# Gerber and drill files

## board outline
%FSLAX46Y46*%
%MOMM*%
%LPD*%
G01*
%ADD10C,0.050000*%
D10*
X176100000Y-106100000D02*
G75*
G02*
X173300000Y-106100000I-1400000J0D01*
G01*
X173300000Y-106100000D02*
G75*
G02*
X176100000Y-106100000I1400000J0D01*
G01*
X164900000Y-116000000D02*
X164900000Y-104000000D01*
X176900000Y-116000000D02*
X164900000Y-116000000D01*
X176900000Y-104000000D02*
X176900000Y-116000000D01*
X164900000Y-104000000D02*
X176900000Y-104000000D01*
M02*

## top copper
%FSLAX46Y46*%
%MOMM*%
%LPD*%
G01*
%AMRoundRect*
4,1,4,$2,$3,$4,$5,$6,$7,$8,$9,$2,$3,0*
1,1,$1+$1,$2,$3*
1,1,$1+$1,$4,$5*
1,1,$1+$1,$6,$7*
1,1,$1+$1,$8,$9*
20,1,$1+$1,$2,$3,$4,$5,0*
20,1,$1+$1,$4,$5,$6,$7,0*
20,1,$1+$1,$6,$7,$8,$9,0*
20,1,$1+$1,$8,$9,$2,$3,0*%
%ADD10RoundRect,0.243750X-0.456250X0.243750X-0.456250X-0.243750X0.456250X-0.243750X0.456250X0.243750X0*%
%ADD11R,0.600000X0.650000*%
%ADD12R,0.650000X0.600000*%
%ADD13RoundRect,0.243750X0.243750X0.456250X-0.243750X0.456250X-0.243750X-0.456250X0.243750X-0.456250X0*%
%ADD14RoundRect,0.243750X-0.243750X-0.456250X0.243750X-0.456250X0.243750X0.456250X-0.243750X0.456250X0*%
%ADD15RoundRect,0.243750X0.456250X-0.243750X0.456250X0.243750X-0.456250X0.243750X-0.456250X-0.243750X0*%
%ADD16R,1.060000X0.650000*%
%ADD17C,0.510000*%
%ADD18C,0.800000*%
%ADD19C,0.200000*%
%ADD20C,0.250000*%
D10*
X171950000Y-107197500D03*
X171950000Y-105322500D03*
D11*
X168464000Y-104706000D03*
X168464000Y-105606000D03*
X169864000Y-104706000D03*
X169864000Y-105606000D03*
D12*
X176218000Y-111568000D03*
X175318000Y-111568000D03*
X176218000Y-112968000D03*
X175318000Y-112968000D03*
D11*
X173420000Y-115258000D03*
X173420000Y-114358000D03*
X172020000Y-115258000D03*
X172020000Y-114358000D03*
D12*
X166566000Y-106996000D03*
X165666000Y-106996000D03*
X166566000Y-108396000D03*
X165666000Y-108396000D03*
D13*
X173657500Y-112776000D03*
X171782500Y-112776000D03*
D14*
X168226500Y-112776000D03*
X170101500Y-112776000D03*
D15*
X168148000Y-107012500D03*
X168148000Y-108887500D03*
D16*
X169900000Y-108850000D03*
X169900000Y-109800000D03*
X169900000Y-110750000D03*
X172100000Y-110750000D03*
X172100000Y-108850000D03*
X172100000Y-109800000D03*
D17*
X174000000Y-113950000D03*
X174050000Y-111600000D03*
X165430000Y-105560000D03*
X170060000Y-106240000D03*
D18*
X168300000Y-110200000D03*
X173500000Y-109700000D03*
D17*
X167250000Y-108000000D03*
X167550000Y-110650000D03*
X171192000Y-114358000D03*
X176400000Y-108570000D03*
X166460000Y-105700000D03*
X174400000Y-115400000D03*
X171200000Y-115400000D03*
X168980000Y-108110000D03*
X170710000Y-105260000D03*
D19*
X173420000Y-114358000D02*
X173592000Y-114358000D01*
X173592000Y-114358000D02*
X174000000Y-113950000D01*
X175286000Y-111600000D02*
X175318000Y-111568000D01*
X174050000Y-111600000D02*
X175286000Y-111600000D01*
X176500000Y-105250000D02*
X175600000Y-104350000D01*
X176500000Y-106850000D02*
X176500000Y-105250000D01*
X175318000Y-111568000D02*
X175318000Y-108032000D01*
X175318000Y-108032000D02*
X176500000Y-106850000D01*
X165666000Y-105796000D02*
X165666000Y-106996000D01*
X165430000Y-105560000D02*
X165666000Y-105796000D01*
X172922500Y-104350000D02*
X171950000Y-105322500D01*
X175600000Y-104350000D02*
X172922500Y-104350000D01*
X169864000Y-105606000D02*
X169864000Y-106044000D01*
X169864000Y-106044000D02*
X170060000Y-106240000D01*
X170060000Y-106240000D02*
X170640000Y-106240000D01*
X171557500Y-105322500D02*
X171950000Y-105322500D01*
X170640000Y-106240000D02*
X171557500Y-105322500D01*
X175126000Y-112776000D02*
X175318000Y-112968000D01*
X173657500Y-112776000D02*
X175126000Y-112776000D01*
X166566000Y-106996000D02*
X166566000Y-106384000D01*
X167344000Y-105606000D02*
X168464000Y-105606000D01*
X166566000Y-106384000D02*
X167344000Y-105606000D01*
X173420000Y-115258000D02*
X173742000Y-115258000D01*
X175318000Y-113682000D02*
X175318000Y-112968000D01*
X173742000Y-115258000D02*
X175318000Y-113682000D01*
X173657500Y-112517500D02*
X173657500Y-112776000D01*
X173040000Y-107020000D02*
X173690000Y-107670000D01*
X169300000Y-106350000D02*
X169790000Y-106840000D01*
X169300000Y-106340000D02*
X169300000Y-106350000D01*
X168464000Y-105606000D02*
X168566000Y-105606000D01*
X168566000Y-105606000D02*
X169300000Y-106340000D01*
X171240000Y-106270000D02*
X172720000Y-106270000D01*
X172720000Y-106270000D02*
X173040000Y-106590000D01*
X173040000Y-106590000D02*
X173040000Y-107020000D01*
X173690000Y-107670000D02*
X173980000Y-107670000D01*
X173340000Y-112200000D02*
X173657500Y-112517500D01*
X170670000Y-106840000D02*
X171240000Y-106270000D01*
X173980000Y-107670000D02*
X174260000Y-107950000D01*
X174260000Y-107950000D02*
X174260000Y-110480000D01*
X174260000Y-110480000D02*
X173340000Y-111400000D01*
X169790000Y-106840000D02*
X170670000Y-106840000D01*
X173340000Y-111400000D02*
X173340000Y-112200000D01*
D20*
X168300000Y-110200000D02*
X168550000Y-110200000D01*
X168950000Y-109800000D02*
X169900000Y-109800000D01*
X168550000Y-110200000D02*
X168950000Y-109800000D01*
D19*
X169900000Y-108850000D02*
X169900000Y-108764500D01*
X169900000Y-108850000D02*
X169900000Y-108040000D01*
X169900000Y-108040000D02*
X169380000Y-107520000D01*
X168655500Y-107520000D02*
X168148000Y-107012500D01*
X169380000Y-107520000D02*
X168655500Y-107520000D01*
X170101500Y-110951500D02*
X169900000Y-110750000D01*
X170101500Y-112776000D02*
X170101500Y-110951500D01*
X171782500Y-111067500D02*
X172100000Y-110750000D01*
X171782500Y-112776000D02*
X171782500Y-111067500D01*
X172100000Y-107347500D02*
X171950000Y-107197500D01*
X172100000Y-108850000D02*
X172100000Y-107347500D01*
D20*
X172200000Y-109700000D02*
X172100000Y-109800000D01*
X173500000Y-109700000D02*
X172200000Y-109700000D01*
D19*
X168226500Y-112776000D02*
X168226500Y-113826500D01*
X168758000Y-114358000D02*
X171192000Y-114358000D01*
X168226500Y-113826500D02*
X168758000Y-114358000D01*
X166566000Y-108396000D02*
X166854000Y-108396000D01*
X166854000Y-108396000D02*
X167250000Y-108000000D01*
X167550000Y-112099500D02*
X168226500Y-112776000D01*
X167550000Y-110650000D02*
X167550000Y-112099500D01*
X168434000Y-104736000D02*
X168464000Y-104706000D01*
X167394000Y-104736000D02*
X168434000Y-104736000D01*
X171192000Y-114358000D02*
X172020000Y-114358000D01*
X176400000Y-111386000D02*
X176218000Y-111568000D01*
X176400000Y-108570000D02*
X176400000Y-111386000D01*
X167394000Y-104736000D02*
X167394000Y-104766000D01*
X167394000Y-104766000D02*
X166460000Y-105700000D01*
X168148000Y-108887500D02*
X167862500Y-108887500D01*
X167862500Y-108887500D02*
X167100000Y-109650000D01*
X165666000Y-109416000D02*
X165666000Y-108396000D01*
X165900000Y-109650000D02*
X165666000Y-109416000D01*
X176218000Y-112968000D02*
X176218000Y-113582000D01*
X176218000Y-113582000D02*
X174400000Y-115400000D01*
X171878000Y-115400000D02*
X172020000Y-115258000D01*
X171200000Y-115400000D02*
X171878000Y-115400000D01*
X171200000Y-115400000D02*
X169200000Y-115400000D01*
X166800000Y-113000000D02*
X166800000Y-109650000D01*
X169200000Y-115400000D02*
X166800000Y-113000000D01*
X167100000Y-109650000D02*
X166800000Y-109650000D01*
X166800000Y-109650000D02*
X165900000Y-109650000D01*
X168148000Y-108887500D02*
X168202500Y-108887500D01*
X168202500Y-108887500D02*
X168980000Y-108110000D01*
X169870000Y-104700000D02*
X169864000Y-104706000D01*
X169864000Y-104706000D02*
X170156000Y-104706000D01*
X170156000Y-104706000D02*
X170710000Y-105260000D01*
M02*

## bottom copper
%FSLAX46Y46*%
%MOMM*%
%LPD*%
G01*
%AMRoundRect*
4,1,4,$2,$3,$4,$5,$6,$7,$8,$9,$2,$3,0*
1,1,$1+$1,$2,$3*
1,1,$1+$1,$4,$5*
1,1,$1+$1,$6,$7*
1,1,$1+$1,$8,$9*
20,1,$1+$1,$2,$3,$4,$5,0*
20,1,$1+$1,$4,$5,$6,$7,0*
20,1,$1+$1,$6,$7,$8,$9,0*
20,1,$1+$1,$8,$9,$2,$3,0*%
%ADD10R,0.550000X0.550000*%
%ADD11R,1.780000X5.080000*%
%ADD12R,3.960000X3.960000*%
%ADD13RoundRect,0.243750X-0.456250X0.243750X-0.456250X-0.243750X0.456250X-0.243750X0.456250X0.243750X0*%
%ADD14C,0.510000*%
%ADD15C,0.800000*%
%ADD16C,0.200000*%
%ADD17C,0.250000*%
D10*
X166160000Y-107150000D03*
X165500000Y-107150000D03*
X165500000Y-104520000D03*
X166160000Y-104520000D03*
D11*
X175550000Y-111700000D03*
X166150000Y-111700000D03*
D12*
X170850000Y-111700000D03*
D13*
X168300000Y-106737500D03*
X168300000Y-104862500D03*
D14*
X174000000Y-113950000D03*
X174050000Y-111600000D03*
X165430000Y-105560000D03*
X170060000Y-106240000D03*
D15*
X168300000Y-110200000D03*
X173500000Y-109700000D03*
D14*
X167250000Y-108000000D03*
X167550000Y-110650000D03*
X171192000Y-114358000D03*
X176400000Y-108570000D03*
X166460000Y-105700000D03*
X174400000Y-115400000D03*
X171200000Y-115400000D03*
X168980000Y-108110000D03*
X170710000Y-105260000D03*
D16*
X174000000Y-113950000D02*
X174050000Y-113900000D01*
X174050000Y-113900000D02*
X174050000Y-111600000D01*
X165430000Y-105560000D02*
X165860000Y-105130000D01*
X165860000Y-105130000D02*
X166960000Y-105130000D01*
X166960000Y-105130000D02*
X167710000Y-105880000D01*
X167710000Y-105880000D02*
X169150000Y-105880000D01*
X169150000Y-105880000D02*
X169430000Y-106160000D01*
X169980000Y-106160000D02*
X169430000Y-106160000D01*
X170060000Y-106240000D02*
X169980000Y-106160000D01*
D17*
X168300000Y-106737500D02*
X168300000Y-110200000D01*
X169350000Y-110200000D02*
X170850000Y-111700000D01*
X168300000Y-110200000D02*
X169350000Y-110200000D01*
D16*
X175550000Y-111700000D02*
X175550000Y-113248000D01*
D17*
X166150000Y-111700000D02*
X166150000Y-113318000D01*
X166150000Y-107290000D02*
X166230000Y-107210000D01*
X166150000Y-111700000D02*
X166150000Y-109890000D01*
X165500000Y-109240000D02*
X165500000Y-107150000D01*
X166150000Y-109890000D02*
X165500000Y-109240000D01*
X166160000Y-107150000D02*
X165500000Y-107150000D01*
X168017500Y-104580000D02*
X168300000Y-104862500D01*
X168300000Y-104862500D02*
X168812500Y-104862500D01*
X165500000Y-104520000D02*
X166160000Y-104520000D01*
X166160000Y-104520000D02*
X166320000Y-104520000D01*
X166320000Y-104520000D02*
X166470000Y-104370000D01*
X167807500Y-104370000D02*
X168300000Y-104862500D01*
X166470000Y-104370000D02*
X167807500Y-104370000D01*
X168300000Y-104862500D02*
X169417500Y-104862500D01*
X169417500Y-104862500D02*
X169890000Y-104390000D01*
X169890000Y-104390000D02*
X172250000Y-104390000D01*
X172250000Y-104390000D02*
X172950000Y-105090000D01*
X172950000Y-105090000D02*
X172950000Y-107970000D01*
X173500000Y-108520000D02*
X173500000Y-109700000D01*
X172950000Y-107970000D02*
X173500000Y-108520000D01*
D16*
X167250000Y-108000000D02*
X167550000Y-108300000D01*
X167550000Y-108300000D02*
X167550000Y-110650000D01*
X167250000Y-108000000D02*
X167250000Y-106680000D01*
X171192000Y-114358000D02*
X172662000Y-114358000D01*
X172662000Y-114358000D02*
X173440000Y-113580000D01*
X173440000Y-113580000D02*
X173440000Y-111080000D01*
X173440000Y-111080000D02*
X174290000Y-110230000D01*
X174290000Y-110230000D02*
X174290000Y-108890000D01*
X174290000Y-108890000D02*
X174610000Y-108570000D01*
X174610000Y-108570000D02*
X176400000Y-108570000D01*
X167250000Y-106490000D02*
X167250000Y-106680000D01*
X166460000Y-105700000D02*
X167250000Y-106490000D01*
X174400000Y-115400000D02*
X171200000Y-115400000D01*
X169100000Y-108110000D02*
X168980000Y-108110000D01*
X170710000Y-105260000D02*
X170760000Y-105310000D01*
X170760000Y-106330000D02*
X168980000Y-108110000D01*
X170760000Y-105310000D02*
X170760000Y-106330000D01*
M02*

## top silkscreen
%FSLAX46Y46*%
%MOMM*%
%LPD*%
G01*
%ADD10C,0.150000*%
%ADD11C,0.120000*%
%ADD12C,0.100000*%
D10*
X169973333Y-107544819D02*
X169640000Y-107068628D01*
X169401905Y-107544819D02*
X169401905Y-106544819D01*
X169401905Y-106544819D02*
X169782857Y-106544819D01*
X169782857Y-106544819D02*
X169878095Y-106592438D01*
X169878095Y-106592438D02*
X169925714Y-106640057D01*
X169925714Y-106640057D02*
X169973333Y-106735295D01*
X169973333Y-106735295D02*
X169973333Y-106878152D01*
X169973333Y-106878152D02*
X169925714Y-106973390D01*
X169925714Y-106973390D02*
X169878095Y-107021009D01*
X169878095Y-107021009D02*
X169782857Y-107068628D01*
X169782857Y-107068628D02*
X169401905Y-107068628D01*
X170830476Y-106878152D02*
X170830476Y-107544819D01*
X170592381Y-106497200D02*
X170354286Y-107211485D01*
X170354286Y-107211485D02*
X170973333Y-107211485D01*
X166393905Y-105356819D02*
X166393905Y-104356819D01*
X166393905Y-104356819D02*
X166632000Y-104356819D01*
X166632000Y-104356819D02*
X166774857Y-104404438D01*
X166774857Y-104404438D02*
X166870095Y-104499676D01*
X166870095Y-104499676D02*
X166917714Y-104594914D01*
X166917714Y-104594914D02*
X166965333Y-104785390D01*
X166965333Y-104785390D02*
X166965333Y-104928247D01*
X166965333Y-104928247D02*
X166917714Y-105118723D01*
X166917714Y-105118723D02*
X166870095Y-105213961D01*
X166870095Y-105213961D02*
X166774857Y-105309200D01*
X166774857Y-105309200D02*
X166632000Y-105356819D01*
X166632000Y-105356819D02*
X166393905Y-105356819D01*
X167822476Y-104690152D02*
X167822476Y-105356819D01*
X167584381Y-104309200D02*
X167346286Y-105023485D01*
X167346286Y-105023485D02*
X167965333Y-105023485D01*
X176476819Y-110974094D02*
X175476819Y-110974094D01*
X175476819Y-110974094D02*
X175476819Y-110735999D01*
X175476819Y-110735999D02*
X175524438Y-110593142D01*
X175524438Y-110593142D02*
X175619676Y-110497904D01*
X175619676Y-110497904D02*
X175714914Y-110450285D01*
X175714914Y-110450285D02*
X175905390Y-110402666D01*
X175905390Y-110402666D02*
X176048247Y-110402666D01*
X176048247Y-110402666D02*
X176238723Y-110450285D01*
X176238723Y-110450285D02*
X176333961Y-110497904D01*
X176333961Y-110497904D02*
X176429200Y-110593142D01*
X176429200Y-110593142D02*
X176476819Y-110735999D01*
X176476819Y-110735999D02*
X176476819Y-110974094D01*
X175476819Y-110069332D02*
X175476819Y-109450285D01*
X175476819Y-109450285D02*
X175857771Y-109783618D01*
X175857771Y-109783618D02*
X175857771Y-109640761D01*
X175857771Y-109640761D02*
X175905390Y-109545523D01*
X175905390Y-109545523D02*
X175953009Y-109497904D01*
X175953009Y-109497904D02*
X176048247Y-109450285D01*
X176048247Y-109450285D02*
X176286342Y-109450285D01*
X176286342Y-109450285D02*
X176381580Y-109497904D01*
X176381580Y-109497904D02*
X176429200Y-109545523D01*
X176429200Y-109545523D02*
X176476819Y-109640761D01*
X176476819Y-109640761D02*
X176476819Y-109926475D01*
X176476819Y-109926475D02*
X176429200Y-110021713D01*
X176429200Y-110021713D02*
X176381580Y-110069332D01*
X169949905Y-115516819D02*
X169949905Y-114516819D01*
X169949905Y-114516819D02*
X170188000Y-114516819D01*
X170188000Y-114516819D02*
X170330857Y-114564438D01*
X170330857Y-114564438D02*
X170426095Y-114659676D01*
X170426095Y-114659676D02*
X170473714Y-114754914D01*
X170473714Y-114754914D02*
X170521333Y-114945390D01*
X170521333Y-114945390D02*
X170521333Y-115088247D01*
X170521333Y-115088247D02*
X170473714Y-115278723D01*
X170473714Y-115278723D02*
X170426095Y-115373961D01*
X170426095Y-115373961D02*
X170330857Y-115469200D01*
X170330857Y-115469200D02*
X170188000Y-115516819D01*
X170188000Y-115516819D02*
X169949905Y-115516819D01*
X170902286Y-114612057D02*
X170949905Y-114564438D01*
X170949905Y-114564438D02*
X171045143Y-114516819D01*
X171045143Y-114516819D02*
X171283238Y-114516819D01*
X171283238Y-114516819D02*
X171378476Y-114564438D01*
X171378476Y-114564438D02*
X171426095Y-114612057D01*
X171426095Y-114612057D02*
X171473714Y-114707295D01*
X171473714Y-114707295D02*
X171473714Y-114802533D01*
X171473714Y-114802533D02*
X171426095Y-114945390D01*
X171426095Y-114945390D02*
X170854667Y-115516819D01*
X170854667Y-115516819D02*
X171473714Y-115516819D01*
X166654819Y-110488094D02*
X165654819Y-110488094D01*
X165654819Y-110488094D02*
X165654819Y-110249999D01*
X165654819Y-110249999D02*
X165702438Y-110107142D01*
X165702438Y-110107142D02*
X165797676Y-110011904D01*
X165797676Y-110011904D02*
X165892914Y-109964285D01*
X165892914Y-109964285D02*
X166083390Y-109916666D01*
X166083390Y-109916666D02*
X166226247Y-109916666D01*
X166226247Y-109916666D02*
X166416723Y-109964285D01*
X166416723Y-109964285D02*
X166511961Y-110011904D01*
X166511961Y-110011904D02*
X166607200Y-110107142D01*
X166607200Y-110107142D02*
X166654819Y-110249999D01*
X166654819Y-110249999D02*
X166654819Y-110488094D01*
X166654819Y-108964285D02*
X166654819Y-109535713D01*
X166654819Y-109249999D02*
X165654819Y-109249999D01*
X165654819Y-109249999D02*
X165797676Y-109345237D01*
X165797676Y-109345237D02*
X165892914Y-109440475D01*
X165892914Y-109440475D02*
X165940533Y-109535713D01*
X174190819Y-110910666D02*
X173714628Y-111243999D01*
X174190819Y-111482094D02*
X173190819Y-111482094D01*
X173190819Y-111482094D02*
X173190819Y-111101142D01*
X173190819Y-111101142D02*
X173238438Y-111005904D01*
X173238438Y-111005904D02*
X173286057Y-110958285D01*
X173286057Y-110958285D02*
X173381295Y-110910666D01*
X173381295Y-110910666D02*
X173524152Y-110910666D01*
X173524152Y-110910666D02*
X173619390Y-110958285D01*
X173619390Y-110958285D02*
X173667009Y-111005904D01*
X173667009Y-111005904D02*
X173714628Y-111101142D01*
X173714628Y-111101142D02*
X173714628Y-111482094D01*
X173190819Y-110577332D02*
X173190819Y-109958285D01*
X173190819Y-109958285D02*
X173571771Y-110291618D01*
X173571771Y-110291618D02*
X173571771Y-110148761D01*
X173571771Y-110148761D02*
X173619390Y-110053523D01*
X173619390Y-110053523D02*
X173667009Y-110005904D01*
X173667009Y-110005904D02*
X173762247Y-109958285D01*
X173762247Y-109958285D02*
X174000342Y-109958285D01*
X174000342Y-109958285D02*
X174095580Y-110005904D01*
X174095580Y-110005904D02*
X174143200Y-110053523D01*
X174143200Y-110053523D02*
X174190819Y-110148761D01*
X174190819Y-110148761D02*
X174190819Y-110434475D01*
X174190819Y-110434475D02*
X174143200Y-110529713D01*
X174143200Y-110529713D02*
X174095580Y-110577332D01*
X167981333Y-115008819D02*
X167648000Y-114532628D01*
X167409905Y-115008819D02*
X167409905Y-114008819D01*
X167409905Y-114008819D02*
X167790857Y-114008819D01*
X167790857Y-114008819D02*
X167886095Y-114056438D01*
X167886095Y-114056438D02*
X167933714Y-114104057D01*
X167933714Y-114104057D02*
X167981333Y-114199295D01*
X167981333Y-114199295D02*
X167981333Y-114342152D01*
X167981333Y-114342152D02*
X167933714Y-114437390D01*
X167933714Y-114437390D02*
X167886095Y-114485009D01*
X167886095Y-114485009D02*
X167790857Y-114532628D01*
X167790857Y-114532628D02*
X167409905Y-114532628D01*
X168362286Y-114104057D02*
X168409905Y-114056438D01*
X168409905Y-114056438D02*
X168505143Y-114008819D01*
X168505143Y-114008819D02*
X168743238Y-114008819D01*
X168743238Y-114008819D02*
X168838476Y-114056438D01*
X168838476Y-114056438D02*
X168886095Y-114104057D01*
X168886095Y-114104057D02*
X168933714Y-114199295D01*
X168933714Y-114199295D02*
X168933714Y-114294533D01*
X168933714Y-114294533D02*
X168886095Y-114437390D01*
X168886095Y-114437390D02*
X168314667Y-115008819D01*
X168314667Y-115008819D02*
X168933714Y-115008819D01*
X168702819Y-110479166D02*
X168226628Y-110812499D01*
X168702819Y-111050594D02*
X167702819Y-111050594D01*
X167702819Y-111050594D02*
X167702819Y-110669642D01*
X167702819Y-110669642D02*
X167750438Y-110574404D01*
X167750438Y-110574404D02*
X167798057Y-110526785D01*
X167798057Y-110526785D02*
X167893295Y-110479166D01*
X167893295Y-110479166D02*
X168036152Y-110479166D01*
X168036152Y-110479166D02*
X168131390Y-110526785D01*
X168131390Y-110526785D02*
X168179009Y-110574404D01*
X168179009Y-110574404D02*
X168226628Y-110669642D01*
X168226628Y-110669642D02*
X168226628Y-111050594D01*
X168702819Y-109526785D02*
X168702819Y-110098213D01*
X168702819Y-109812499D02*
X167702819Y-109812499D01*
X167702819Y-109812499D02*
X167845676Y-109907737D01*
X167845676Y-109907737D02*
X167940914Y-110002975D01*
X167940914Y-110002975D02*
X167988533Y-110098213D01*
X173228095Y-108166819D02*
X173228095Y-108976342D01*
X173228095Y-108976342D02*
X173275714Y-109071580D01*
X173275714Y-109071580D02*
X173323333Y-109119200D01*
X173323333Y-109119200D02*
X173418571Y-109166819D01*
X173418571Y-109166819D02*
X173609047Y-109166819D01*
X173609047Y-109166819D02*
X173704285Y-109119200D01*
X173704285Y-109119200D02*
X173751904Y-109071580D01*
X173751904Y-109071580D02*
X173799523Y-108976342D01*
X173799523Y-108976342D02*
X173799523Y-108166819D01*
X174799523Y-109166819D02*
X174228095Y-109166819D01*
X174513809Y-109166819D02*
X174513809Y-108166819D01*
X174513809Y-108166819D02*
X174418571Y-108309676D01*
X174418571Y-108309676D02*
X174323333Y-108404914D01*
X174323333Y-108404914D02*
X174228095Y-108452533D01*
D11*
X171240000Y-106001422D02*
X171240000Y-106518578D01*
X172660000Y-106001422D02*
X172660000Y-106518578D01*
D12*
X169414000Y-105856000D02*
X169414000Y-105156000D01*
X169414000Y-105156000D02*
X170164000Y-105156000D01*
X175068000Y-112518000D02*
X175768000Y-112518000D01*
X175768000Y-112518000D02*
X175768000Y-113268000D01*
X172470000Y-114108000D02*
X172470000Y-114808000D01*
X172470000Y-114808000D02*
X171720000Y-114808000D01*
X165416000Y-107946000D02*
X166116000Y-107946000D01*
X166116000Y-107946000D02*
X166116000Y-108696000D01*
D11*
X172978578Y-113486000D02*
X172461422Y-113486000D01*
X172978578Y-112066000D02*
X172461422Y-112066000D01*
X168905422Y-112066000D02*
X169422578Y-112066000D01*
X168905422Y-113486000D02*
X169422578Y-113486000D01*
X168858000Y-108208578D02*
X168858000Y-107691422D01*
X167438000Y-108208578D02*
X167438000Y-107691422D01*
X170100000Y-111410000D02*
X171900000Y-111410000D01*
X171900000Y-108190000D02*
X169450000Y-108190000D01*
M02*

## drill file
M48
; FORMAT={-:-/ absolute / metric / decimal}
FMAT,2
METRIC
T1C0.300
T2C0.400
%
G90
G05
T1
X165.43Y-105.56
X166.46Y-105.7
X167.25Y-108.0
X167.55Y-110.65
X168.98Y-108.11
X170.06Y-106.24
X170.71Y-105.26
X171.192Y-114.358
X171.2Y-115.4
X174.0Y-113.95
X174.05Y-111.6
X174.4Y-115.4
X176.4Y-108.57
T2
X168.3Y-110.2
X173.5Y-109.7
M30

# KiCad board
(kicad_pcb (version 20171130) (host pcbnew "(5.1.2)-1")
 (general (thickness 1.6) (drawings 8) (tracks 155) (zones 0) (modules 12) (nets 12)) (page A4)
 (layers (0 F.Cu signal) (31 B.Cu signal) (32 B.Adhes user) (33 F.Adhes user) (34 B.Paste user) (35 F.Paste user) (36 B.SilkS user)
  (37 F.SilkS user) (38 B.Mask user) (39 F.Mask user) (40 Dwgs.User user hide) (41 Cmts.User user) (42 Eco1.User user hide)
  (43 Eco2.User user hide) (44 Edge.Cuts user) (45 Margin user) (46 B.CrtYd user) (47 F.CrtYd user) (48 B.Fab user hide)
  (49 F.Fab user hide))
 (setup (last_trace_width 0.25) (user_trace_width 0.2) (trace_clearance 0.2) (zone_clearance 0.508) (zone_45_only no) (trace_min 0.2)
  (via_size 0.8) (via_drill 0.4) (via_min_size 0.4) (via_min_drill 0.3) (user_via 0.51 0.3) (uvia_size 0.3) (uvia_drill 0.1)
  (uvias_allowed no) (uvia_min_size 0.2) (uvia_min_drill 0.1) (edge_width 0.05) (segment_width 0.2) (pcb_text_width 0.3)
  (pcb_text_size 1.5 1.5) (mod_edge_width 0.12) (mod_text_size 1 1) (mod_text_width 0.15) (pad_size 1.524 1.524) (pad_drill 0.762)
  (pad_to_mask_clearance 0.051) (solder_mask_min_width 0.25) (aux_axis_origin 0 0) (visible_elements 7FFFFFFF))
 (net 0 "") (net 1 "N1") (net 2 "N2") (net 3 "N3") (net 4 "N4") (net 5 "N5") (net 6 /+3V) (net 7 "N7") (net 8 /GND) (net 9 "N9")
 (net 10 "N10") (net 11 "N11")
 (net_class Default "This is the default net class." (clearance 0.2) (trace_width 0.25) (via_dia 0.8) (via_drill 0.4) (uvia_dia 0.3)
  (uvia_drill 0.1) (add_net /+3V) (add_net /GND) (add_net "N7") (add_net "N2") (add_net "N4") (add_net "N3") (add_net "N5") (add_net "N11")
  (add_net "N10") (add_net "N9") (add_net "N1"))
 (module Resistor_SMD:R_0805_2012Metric (layer F.Cu) (at 171.95 106.26 270)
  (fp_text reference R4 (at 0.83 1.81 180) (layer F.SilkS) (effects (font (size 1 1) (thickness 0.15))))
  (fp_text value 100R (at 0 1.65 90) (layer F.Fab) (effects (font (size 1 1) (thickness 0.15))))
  (fp_line (start -0.258578 0.71) (end 0.258578 0.71) (layer F.SilkS) (width 0.12))
  (fp_line (start -0.258578 -0.71) (end 0.258578 -0.71) (layer F.SilkS) (width 0.12))
  (pad 2 smd roundrect (at 0.9375 0 270) (size 0.975 1.4) (layers F.Cu F.Paste F.Mask) (roundrect_rratio 0.25) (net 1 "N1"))
  (pad 1 smd roundrect (at -0.9375 0 270) (size 0.975 1.4) (layers F.Cu F.Paste F.Mask) (roundrect_rratio 0.25) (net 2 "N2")))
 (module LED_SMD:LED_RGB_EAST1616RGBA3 (layer F.Cu) (at 169.164 105.156)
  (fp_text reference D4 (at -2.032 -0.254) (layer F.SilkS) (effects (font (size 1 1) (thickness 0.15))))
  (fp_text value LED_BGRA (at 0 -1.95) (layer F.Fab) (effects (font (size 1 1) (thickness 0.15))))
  (fp_line (start 0.25 0.7) (end 0.25 0) (layer F.SilkS) (width 0.1))
  (fp_line (start 0.25 0) (end 1 0) (layer F.SilkS) (width 0.1))
  (pad 2 smd rect (at -0.7 -0.45) (size 0.6 0.65) (layers F.Cu F.Paste F.Mask) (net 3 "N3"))
  (pad 1 smd rect (at -0.7 0.45) (size 0.6 0.65) (layers F.Cu F.Paste F.Mask) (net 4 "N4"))
  (pad 3 smd rect (at 0.7 -0.45) (size 0.6 0.65) (layers F.Cu F.Paste F.Mask) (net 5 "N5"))
  (pad 4 smd rect (at 0.7 0.45) (size 0.6 0.65) (layers F.Cu F.Paste F.Mask) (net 2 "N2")))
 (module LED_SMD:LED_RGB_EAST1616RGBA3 (layer F.Cu) (at 175.768 112.268 270)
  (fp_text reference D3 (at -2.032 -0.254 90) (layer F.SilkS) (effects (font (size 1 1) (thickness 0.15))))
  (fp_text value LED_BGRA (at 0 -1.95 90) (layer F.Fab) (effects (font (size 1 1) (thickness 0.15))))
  (fp_line (start 0.25 0.7) (end 0.25 0) (layer F.SilkS) (width 0.1))
  (fp_line (start 0.25 0) (end 1 0) (layer F.SilkS) (width 0.1))
  (pad 2 smd rect (at -0.7 -0.45 270) (size 0.6 0.65) (layers F.Cu F.Paste F.Mask) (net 3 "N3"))
  (pad 1 smd rect (at -0.7 0.45 270) (size 0.6 0.65) (layers F.Cu F.Paste F.Mask) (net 2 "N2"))
  (pad 3 smd rect (at 0.7 -0.45 270) (size 0.6 0.65) (layers F.Cu F.Paste F.Mask) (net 5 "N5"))
  (pad 4 smd rect (at 0.7 0.45 270) (size 0.6 0.65) (layers F.Cu F.Paste F.Mask) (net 4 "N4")))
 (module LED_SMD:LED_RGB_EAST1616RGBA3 (layer F.Cu) (at 172.72 114.808 180)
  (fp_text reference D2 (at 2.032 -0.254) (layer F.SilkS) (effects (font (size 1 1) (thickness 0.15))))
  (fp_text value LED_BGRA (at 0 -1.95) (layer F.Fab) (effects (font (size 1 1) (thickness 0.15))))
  (fp_line (start 0.25 0.7) (end 0.25 0) (layer F.SilkS) (width 0.1))
  (fp_line (start 0.25 0) (end 1 0) (layer F.SilkS) (width 0.1))
  (pad 2 smd rect (at -0.7 -0.45 180) (size 0.6 0.65) (layers F.Cu F.Paste F.Mask) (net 4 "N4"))
  (pad 1 smd rect (at -0.7 0.45 180) (size 0.6 0.65) (layers F.Cu F.Paste F.Mask) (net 2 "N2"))
  (pad 3 smd rect (at 0.7 -0.45 180) (size 0.6 0.65) (layers F.Cu F.Paste F.Mask) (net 5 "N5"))
  (pad 4 smd rect (at 0.7 0.45 180) (size 0.6 0.65) (layers F.Cu F.Paste F.Mask) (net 3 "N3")))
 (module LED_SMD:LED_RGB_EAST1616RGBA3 (layer F.Cu) (at 166.116 107.696 270)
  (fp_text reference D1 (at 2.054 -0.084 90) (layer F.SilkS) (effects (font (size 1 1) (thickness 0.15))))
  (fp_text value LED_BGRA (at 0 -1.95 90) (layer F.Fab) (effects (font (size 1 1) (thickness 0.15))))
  (fp_line (start 0.25 0.7) (end 0.25 0) (layer F.SilkS) (width 0.1))
  (fp_line (start 0.25 0) (end 1 0) (layer F.SilkS) (width 0.1))
  (pad 2 smd rect (at -0.7 -0.45 270) (size 0.6 0.65) (layers F.Cu F.Paste F.Mask) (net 4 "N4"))
  (pad 1 smd rect (at -0.7 0.45 270) (size 0.6 0.65) (layers F.Cu F.Paste F.Mask) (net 2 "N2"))
  (pad 3 smd rect (at 0.7 -0.45 270) (size 0.6 0.65) (layers F.Cu F.Paste F.Mask) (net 3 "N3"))
  (pad 4 smd rect (at 0.7 0.45 270) (size 0.6 0.65) (layers F.Cu F.Paste F.Mask) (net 5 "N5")))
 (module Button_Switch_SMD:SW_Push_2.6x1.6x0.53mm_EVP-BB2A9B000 (layer B.Cu) (at 165.83 105.84 90)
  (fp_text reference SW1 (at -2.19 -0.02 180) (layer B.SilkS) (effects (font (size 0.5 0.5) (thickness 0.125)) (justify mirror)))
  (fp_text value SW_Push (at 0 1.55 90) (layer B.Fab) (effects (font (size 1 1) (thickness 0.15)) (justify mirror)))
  (pad 1 smd rect (at -1.31 0.33 90) (size 0.55 0.55) (layers B.Cu B.Paste B.Mask) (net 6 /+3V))
  (pad 1 smd rect (at -1.31 -0.33 90) (size 0.55 0.55) (layers B.Cu B.Paste B.Mask) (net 6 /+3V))
  (pad 2 smd rect (at 1.32 -0.33 90) (size 0.55 0.55) (layers B.Cu B.Paste B.Mask) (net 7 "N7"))
  (pad 2 smd rect (at 1.32 0.33 90) (size 0.55 0.55) (layers B.Cu B.Paste B.Mask) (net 7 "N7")))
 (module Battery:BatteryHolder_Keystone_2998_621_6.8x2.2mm (layer B.Cu) (at 170.85 111.7)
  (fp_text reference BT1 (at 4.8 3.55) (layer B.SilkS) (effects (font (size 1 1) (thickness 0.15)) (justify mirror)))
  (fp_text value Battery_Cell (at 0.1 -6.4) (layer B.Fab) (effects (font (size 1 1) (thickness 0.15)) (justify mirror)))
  (pad 1 smd rect (at 4.7 0) (size 1.78 5.08) (layers B.Cu B.Paste B.Mask) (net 6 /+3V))
  (pad 1 smd rect (at -4.7 0) (size 1.78 5.08) (layers B.Cu B.Paste B.Mask) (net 6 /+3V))
  (pad 2 smd rect (at 0 0) (size 3.96 3.96) (layers B.Cu B.Paste B.Mask) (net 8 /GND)))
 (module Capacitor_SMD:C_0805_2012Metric (layer B.Cu) (at 168.3 105.8 270)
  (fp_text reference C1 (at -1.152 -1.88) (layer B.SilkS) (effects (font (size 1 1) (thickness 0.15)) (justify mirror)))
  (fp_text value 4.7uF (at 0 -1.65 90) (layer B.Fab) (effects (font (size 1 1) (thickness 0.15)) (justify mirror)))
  (pad 2 smd roundrect (at 0.9375 0 270) (size 0.975 1.4) (layers B.Cu B.Paste B.Mask) (roundrect_rratio 0.25) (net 8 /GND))
  (pad 1 smd roundrect (at -0.9375 0 270) (size 0.975 1.4) (layers B.Cu B.Paste B.Mask) (roundrect_rratio 0.25) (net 7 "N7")))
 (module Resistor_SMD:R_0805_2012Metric (layer F.Cu) (at 172.72 112.776 180)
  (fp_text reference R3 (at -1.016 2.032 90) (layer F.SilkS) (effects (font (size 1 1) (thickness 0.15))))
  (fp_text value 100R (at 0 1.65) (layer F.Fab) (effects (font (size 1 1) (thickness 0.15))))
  (fp_line (start -0.258578 -0.71) (end 0.258578 -0.71) (layer F.SilkS) (width 0.12))
  (fp_line (start -0.258578 0.71) (end 0.258578 0.71) (layer F.SilkS) (width 0.12))
  (pad 1 smd roundrect (at -0.9375 0 180) (size 0.975 1.4) (layers F.Cu F.Paste F.Mask) (roundrect_rratio 0.25) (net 4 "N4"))
  (pad 2 smd roundrect (at 0.9375 0 180) (size 0.975 1.4) (layers F.Cu F.Paste F.Mask) (roundrect_rratio 0.25) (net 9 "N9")))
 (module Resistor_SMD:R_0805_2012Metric (layer F.Cu) (at 169.164 112.776)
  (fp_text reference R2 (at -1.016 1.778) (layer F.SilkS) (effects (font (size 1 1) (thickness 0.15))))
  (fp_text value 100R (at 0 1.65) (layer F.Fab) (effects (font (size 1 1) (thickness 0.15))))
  (fp_line (start -0.258578 -0.71) (end 0.258578 -0.71) (layer F.SilkS) (width 0.12))
  (fp_line (start -0.258578 0.71) (end 0.258578 0.71) (layer F.SilkS) (width 0.12))
  (pad 1 smd roundrect (at -0.9375 0) (size 0.975 1.4) (layers F.Cu F.Paste F.Mask) (roundrect_rratio 0.25) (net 3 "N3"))
  (pad 2 smd roundrect (at 0.9375 0) (size 0.975 1.4) (layers F.Cu F.Paste F.Mask) (roundrect_rratio 0.25) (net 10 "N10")))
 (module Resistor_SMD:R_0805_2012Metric (layer F.Cu) (at 168.148 107.95 90)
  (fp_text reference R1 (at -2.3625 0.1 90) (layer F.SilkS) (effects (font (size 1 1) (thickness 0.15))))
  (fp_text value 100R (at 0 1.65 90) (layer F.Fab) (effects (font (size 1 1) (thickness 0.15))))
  (fp_line (start -0.258578 0.71) (end 0.258578 0.71) (layer F.SilkS) (width 0.12))
  (fp_line (start -0.258578 -0.71) (end 0.258578 -0.71) (layer F.SilkS) (width 0.12))
  (pad 2 smd roundrect (at 0.9375 0 90) (size 0.975 1.4) (layers F.Cu F.Paste F.Mask) (roundrect_rratio 0.25) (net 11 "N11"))
  (pad 1 smd roundrect (at -0.9375 0 90) (size 0.975 1.4) (layers F.Cu F.Paste F.Mask) (roundrect_rratio 0.25) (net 5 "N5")))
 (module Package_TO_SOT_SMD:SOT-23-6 (layer F.Cu) (at 171 109.8)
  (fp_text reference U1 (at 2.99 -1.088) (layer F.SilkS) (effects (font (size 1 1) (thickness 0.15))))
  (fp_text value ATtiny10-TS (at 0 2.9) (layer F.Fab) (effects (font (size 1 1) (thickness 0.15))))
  (fp_line (start -0.9 1.61) (end 0.9 1.61) (layer F.SilkS) (width 0.12))
  (fp_line (start 0.9 -1.61) (end -1.55 -1.61) (layer F.SilkS) (width 0.12))
  (pad 1 smd rect (at -1.1 -0.95) (size 1.06 0.65) (layers F.Cu F.Paste F.Mask) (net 11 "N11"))
  (pad 2 smd rect (at -1.1 0) (size 1.06 0.65) (layers F.Cu F.Paste F.Mask) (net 8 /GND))
  (pad 3 smd rect (at -1.1 0.95) (size 1.06 0.65) (layers F.Cu F.Paste F.Mask) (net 10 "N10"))
  (pad 4 smd rect (at 1.1 0.95) (size 1.06 0.65) (layers F.Cu F.Paste F.Mask) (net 9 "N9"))
  (pad 6 smd rect (at 1.1 -0.95) (size 1.06 0.65) (layers F.Cu F.Paste F.Mask) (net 1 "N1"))
  (pad 5 smd rect (at 1.1 0) (size 1.06 0.65) (layers F.Cu F.Paste F.Mask) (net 7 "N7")))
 (gr_circle (center 174.7 106.1) (end 176.1 106.1) (layer Edge.Cuts) (width 0.05))
 (gr_line (start 164.9 116) (end 164.9 104) (layer Edge.Cuts) (width 0.05))
 (gr_line (start 176.9 116) (end 164.9 116) (layer Edge.Cuts) (width 0.05))
 (gr_line (start 176.9 104) (end 176.9 116) (layer Edge.Cuts) (width 0.05))
 (gr_line (start 164.9 104) (end 176.9 104) (layer Edge.Cuts) (width 0.05))
 (via (at 174 113.95) (size 0.51) (drill 0.3) (layers F.Cu B.Cu) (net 2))
 (segment (start 173.42 114.358) (end 173.592 114.358) (width 0.2) (layer F.Cu) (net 2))
 (segment (start 173.592 114.358) (end 174 113.95) (width 0.2) (layer F.Cu) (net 2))
 (via (at 174.05 111.6) (size 0.51) (drill 0.3) (layers F.Cu B.Cu) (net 2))
 (segment (start 174 113.95) (end 174.05 113.9) (width 0.2) (layer B.Cu) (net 2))
 (segment (start 174.05 113.9) (end 174.05 111.6) (width 0.2) (layer B.Cu) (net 2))
 (segment (start 175.286 111.6) (end 175.318 111.568) (width 0.2) (layer F.Cu) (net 2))
 (segment (start 174.05 111.6) (end 175.286 111.6) (width 0.2) (layer F.Cu) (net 2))
 (segment (start 176.5 105.25) (end 175.6 104.35) (width 0.2) (layer F.Cu) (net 2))
 (segment (start 176.5 106.85) (end 176.5 105.25) (width 0.2) (layer F.Cu) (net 2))
 (segment (start 175.318 111.568) (end 175.318 108.032) (width 0.2) (layer F.Cu) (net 2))
 (segment (start 175.318 108.032) (end 176.5 106.85) (width 0.2) (layer F.Cu) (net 2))
 (via (at 165.43 105.56) (size 0.51) (drill 0.3) (layers F.Cu B.Cu) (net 2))
 (segment (start 165.666 105.796) (end 165.666 106.996) (width 0.2) (layer F.Cu) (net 2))
 (segment (start 165.43 105.56) (end 165.666 105.796) (width 0.2) (layer F.Cu) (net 2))
 (segment (start 172.9225 104.35) (end 171.95 105.3225) (width 0.2) (layer F.Cu) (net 2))
 (segment (start 175.6 104.35) (end 172.9225 104.35) (width 0.2) (layer F.Cu) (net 2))
 (segment (start 165.43 105.56) (end 165.86 105.13) (width 0.2) (layer B.Cu) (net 2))
 (segment (start 165.86 105.13) (end 166.96 105.13) (width 0.2) (layer B.Cu) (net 2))
 (segment (start 166.96 105.13) (end 167.71 105.88) (width 0.2) (layer B.Cu) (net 2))
 (segment (start 167.71 105.88) (end 169.15 105.88) (width 0.2) (layer B.Cu) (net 2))
 (segment (start 169.15 105.88) (end 169.43 106.16) (width 0.2) (layer B.Cu) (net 2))
 (via (at 170.06 106.24) (size 0.51) (drill 0.3) (layers F.Cu B.Cu) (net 2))
 (segment (start 169.864 105.606) (end 169.864 106.044) (width 0.2) (layer F.Cu) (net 2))
 (segment (start 169.864 106.044) (end 170.06 106.24) (width 0.2) (layer F.Cu) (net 2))
 (segment (start 169.98 106.16) (end 169.43 106.16) (width 0.2) (layer B.Cu) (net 2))
 (segment (start 170.06 106.24) (end 169.98 106.16) (width 0.2) (layer B.Cu) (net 2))
 (segment (start 170.06 106.24) (end 170.64 106.24) (width 0.2) (layer F.Cu) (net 2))
 (segment (start 171.5575 105.3225) (end 171.95 105.3225) (width 0.2) (layer F.Cu) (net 2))
 (segment (start 170.64 106.24) (end 171.5575 105.3225) (width 0.2) (layer F.Cu) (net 2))
 (segment (start 175.126 112.776) (end 175.318 112.968) (width 0.2) (layer F.Cu) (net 4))
 (segment (start 173.6575 112.776) (end 175.126 112.776) (width 0.2) (layer F.Cu) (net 4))
 (segment (start 166.566 106.996) (end 166.566 106.384) (width 0.2) (layer F.Cu) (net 4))
 (segment (start 167.344 105.606) (end 168.464 105.606) (width 0.2) (layer F.Cu) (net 4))
 (segment (start 166.566 106.384) (end 167.344 105.606) (width 0.2) (layer F.Cu) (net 4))
 (segment (start 173.42 115.258) (end 173.742 115.258) (width 0.2) (layer F.Cu) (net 4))
 (segment (start 175.318 113.682) (end 175.318 112.968) (width 0.2) (layer F.Cu) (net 4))
 (segment (start 173.742 115.258) (end 175.318 113.682) (width 0.2) (layer F.Cu) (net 4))
 (segment (start 173.6575 112.5175) (end 173.6575 112.776) (width 0.2) (layer F.Cu) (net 4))
 (segment (start 173.04 107.02) (end 173.69 107.67) (width 0.2) (layer F.Cu) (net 4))
 (segment (start 169.3 106.35) (end 169.79 106.84) (width 0.2) (layer F.Cu) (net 4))
 (segment (start 169.3 106.34) (end 169.3 106.35) (width 0.2) (layer F.Cu) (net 4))
 (segment (start 168.464 105.606) (end 168.566 105.606) (width 0.2) (layer F.Cu) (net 4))
 (segment (start 168.566 105.606) (end 169.3 106.34) (width 0.2) (layer F.Cu) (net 4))
 (segment (start 171.24 106.27) (end 172.72 106.27) (width 0.2) (layer F.Cu) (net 4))
 (segment (start 172.72 106.27) (end 173.04 106.59) (width 0.2) (layer F.Cu) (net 4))
 (segment (start 173.04 106.59) (end 173.04 107.02) (width 0.2) (layer F.Cu) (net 4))
 (segment (start 173.69 107.67) (end 173.98 107.67) (width 0.2) (layer F.Cu) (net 4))
 (segment (start 173.34 112.2) (end 173.6575 112.5175) (width 0.2) (layer F.Cu) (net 4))
 (segment (start 170.67 106.84) (end 171.24 106.27) (width 0.2) (layer F.Cu) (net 4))
 (segment (start 173.98 107.67) (end 174.26 107.95) (width 0.2) (layer F.Cu) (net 4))
 (segment (start 174.26 107.95) (end 174.26 110.48) (width 0.2) (layer F.Cu) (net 4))
 (segment (start 174.26 110.48) (end 173.34 111.4) (width 0.2) (layer F.Cu) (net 4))
 (segment (start 169.79 106.84) (end 170.67 106.84) (width 0.2) (layer F.Cu) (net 4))
 (segment (start 173.34 111.4) (end 173.34 112.2) (width 0.2) (layer F.Cu) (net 4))
 (via (at 168.3 110.2) (size 0.8) (drill 0.4) (layers F.Cu B.Cu) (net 8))
 (segment (start 168.3 106.7375) (end 168.3 110.2) (width 0.25) (layer B.Cu) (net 8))
 (segment (start 168.3 110.2) (end 168.55 110.2) (width 0.25) (layer F.Cu) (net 8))
 (segment (start 168.95 109.8) (end 169.9 109.8) (width 0.25) (layer F.Cu) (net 8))
 (segment (start 168.55 110.2) (end 168.95 109.8) (width 0.25) (layer F.Cu) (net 8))
 (segment (start 169.35 110.2) (end 170.85 111.7) (width 0.25) (layer B.Cu) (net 8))
 (segment (start 168.3 110.2) (end 169.35 110.2) (width 0.25) (layer B.Cu) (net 8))
 (segment (start 169.9 108.85) (end 169.9 108.7645) (width 0.2) (layer F.Cu) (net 11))
 (segment (start 169.9 108.85) (end 169.9 108.04) (width 0.2) (layer F.Cu) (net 11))
 (segment (start 169.9 108.04) (end 169.38 107.52) (width 0.2) (layer F.Cu) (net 11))
 (segment (start 168.6555 107.52) (end 168.148 107.0125) (width 0.2) (layer F.Cu) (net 11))
 (segment (start 169.38 107.52) (end 168.6555 107.52) (width 0.2) (layer F.Cu) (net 11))
 (segment (start 170.1015 110.9515) (end 169.9 110.75) (width 0.2) (layer F.Cu) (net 10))
 (segment (start 170.1015 112.776) (end 170.1015 110.9515) (width 0.2) (layer F.Cu) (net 10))
 (segment (start 171.7825 111.0675) (end 172.1 110.75) (width 0.2) (layer F.Cu) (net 9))
 (segment (start 171.7825 112.776) (end 171.7825 111.0675) (width 0.2) (layer F.Cu) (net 9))
 (segment (start 172.1 107.3475) (end 171.95 107.1975) (width 0.2) (layer F.Cu) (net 1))
 (segment (start 172.1 108.85) (end 172.1 107.3475) (width 0.2) (layer F.Cu) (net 1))
 (segment (start 175.55 111.7) (end 175.55 113.248) (width 0.2) (layer B.Cu) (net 6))
 (segment (start 166.15 111.7) (end 166.15 113.318) (width 0.25) (layer B.Cu) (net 6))
 (segment (start 166.15 107.29) (end 166.23 107.21) (width 0.25) (layer B.Cu) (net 6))
 (segment (start 166.15 111.7) (end 166.15 109.89) (width 0.25) (layer B.Cu) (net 6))
 (segment (start 165.5 109.24) (end 165.5 107.15) (width 0.25) (layer B.Cu) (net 6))
 (segment (start 166.15 109.89) (end 165.5 109.24) (width 0.25) (layer B.Cu) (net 6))
 (segment (start 166.16 107.15) (end 165.5 107.15) (width 0.25) (layer B.Cu) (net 6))
 (segment (start 168.0175 104.58) (end 168.3 104.8625) (width 0.25) (layer B.Cu) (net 7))
 (via (at 173.5 109.7) (size 0.8) (drill 0.4) (layers F.Cu B.Cu) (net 7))
 (segment (start 172.2 109.7) (end 172.1 109.8) (width 0.25) (layer F.Cu) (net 7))
 (segment (start 173.5 109.7) (end 172.2 109.7) (width 0.25) (layer F.Cu) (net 7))
 (segment (start 168.3 104.8625) (end 168.8125 104.8625) (width 0.25) (layer B.Cu) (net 7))
 (segment (start 165.5 104.52) (end 166.16 104.52) (width 0.25) (layer B.Cu) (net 7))
 (segment (start 166.16 104.52) (end 166.32 104.52) (width 0.25) (layer B.Cu) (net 7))
 (segment (start 166.32 104.52) (end 166.47 104.37) (width 0.25) (layer B.Cu) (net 7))
 (segment (start 167.8075 104.37) (end 168.3 104.8625) (width 0.25) (layer B.Cu) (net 7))
 (segment (start 166.47 104.37) (end 167.8075 104.37) (width 0.25) (layer B.Cu) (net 7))
 (segment (start 168.3 104.8625) (end 169.4175 104.8625) (width 0.25) (layer B.Cu) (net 7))
 (segment (start 169.4175 104.8625) (end 169.89 104.39) (width 0.25) (layer B.Cu) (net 7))
 (segment (start 169.89 104.39) (end 172.25 104.39) (width 0.25) (layer B.Cu) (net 7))
 (segment (start 172.25 104.39) (end 172.95 105.09) (width 0.25) (layer B.Cu) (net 7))
 (segment (start 172.95 105.09) (end 172.95 107.97) (width 0.25) (layer B.Cu) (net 7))
 (segment (start 173.5 108.52) (end 173.5 109.7) (width 0.25) (layer B.Cu) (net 7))
 (segment (start 172.95 107.97) (end 173.5 108.52) (width 0.25) (layer B.Cu) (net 7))
 (segment (start 168.2265 112.776) (end 168.2265 113.8265) (width 0.2) (layer F.Cu) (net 3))
 (segment (start 168.758 114.358) (end 171.192 114.358) (width 0.2) (layer F.Cu) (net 3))
 (segment (start 168.2265 113.8265) (end 168.758 114.358) (width 0.2) (layer F.Cu) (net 3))
 (via (at 167.25 108) (size 0.51) (drill 0.3) (layers F.Cu B.Cu) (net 3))
 (segment (start 166.566 108.396) (end 166.854 108.396) (width 0.2) (layer F.Cu) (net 3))
 (segment (start 166.854 108.396) (end 167.25 108) (width 0.2) (layer F.Cu) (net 3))
 (via (at 167.55 110.65) (size 0.51) (drill 0.3) (layers F.Cu B.Cu) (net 3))
 (segment (start 167.25 108) (end 167.55 108.3) (width 0.2) (layer B.Cu) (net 3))
 (segment (start 167.55 108.3) (end 167.55 110.65) (width 0.2) (layer B.Cu) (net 3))
 (segment (start 167.55 112.0995) (end 168.2265 112.776) (width 0.2) (layer F.Cu) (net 3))
 (segment (start 167.55 110.65) (end 167.55 112.0995) (width 0.2) (layer F.Cu) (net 3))
 (segment (start 167.25 108) (end 167.25 106.68) (width 0.2) (layer B.Cu) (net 3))
 (segment (start 168.434 104.736) (end 168.464 104.706) (width 0.2) (layer F.Cu) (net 3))
 (segment (start 167.394 104.736) (end 168.434 104.736) (width 0.2) (layer F.Cu) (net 3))
 (segment (start 171.192 114.358) (end 172.02 114.358) (width 0.2) (layer F.Cu) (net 3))
 (via (at 171.192 114.358) (size 0.51) (drill 0.3) (layers F.Cu B.Cu) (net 3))
 (segment (start 171.192 114.358) (end 172.662 114.358) (width 0.2) (layer B.Cu) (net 3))
 (segment (start 172.662 114.358) (end 173.44 113.58) (width 0.2) (layer B.Cu) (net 3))
 (segment (start 173.44 113.58) (end 173.44 111.08) (width 0.2) (layer B.Cu) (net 3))
 (segment (start 173.44 111.08) (end 174.29 110.23) (width 0.2) (layer B.Cu) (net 3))
 (segment (start 174.29 110.23) (end 174.29 108.89) (width 0.2) (layer B.Cu) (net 3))
 (via (at 176.4 108.57) (size 0.51) (drill 0.3) (layers F.Cu B.Cu) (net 3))
 (segment (start 174.29 108.89) (end 174.61 108.57) (width 0.2) (layer B.Cu) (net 3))
 (segment (start 174.61 108.57) (end 176.4 108.57) (width 0.2) (layer B.Cu) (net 3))
 (segment (start 176.4 111.386) (end 176.218 111.568) (width 0.2) (layer F.Cu) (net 3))
 (segment (start 176.4 108.57) (end 176.4 111.386) (width 0.2) (layer F.Cu) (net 3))
 (via (at 166.46 105.7) (size 0.51) (drill 0.3) (layers F.Cu B.Cu) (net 3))
 (segment (start 167.394 104.736) (end 167.394 104.766) (width 0.2) (layer F.Cu) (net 3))
 (segment (start 167.394 104.766) (end 166.46 105.7) (width 0.2) (layer F.Cu) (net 3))
 (segment (start 167.25 106.49) (end 167.25 106.68) (width 0.2) (layer B.Cu) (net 3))
 (segment (start 166.46 105.7) (end 167.25 106.49) (width 0.2) (layer B.Cu) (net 3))
 (segment (start 168.148 108.8875) (end 167.8625 108.8875) (width 0.2) (layer F.Cu) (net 5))
 (segment (start 167.8625 108.8875) (end 167.1 109.65) (width 0.2) (layer F.Cu) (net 5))
 (segment (start 165.666 109.416) (end 165.666 108.396) (width 0.2) (layer F.Cu) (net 5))
 (segment (start 165.9 109.65) (end 165.666 109.416) (width 0.2) (layer F.Cu) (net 5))
 (via (at 174.4 115.4) (size 0.51) (drill 0.3) (layers F.Cu B.Cu) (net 5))
 (segment (start 176.218 112.968) (end 176.218 113.582) (width 0.2) (layer F.Cu) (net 5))
 (segment (start 176.218 113.582) (end 174.4 115.4) (width 0.2) (layer F.Cu) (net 5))
 (via (at 171.2 115.4) (size 0.51) (drill 0.3) (layers F.Cu B.Cu) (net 5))
 (segment (start 174.4 115.4) (end 171.2 115.4) (width 0.2) (layer B.Cu) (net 5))
 (segment (start 171.878 115.4) (end 172.02 115.258) (width 0.2) (layer F.Cu) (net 5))
 (segment (start 171.2 115.4) (end 171.878 115.4) (width 0.2) (layer F.Cu) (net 5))
 (segment (start 171.2 115.4) (end 169.2 115.4) (width 0.2) (layer F.Cu) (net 5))
 (segment (start 166.8 113) (end 166.8 109.65) (width 0.2) (layer F.Cu) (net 5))
 (segment (start 169.2 115.4) (end 166.8 113) (width 0.2) (layer F.Cu) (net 5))
 (segment (start 167.1 109.65) (end 166.8 109.65) (width 0.2) (layer F.Cu) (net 5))
 (segment (start 166.8 109.65) (end 165.9 109.65) (width 0.2) (layer F.Cu) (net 5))
 (via (at 168.98 108.11) (size 0.51) (drill 0.3) (layers F.Cu B.Cu) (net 5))
 (segment (start 168.148 108.8875) (end 168.2025 108.8875) (width 0.2) (layer F.Cu) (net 5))
 (segment (start 168.2025 108.8875) (end 168.98 108.11) (width 0.2) (layer F.Cu) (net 5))
 (segment (start 169.87 104.7) (end 169.864 104.706) (width 0.2) (layer F.Cu) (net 5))
 (segment (start 169.1 108.11) (end 168.98 108.11) (width 0.2) (layer B.Cu) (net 5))
 (via (at 170.71 105.26) (size 0.51) (drill 0.3) (layers F.Cu B.Cu) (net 5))
 (segment (start 169.864 104.706) (end 170.156 104.706) (width 0.2) (layer F.Cu) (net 5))
 (segment (start 170.156 104.706) (end 170.71 105.26) (width 0.2) (layer F.Cu) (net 5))
 (segment (start 170.71 105.26) (end 170.76 105.31) (width 0.2) (layer B.Cu) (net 5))
 (segment (start 170.76 106.33) (end 168.98 108.11) (width 0.2) (layer B.Cu) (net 5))
 (segment (start 170.76 105.31) (end 170.76 106.33) (width 0.2) (layer B.Cu) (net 5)))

